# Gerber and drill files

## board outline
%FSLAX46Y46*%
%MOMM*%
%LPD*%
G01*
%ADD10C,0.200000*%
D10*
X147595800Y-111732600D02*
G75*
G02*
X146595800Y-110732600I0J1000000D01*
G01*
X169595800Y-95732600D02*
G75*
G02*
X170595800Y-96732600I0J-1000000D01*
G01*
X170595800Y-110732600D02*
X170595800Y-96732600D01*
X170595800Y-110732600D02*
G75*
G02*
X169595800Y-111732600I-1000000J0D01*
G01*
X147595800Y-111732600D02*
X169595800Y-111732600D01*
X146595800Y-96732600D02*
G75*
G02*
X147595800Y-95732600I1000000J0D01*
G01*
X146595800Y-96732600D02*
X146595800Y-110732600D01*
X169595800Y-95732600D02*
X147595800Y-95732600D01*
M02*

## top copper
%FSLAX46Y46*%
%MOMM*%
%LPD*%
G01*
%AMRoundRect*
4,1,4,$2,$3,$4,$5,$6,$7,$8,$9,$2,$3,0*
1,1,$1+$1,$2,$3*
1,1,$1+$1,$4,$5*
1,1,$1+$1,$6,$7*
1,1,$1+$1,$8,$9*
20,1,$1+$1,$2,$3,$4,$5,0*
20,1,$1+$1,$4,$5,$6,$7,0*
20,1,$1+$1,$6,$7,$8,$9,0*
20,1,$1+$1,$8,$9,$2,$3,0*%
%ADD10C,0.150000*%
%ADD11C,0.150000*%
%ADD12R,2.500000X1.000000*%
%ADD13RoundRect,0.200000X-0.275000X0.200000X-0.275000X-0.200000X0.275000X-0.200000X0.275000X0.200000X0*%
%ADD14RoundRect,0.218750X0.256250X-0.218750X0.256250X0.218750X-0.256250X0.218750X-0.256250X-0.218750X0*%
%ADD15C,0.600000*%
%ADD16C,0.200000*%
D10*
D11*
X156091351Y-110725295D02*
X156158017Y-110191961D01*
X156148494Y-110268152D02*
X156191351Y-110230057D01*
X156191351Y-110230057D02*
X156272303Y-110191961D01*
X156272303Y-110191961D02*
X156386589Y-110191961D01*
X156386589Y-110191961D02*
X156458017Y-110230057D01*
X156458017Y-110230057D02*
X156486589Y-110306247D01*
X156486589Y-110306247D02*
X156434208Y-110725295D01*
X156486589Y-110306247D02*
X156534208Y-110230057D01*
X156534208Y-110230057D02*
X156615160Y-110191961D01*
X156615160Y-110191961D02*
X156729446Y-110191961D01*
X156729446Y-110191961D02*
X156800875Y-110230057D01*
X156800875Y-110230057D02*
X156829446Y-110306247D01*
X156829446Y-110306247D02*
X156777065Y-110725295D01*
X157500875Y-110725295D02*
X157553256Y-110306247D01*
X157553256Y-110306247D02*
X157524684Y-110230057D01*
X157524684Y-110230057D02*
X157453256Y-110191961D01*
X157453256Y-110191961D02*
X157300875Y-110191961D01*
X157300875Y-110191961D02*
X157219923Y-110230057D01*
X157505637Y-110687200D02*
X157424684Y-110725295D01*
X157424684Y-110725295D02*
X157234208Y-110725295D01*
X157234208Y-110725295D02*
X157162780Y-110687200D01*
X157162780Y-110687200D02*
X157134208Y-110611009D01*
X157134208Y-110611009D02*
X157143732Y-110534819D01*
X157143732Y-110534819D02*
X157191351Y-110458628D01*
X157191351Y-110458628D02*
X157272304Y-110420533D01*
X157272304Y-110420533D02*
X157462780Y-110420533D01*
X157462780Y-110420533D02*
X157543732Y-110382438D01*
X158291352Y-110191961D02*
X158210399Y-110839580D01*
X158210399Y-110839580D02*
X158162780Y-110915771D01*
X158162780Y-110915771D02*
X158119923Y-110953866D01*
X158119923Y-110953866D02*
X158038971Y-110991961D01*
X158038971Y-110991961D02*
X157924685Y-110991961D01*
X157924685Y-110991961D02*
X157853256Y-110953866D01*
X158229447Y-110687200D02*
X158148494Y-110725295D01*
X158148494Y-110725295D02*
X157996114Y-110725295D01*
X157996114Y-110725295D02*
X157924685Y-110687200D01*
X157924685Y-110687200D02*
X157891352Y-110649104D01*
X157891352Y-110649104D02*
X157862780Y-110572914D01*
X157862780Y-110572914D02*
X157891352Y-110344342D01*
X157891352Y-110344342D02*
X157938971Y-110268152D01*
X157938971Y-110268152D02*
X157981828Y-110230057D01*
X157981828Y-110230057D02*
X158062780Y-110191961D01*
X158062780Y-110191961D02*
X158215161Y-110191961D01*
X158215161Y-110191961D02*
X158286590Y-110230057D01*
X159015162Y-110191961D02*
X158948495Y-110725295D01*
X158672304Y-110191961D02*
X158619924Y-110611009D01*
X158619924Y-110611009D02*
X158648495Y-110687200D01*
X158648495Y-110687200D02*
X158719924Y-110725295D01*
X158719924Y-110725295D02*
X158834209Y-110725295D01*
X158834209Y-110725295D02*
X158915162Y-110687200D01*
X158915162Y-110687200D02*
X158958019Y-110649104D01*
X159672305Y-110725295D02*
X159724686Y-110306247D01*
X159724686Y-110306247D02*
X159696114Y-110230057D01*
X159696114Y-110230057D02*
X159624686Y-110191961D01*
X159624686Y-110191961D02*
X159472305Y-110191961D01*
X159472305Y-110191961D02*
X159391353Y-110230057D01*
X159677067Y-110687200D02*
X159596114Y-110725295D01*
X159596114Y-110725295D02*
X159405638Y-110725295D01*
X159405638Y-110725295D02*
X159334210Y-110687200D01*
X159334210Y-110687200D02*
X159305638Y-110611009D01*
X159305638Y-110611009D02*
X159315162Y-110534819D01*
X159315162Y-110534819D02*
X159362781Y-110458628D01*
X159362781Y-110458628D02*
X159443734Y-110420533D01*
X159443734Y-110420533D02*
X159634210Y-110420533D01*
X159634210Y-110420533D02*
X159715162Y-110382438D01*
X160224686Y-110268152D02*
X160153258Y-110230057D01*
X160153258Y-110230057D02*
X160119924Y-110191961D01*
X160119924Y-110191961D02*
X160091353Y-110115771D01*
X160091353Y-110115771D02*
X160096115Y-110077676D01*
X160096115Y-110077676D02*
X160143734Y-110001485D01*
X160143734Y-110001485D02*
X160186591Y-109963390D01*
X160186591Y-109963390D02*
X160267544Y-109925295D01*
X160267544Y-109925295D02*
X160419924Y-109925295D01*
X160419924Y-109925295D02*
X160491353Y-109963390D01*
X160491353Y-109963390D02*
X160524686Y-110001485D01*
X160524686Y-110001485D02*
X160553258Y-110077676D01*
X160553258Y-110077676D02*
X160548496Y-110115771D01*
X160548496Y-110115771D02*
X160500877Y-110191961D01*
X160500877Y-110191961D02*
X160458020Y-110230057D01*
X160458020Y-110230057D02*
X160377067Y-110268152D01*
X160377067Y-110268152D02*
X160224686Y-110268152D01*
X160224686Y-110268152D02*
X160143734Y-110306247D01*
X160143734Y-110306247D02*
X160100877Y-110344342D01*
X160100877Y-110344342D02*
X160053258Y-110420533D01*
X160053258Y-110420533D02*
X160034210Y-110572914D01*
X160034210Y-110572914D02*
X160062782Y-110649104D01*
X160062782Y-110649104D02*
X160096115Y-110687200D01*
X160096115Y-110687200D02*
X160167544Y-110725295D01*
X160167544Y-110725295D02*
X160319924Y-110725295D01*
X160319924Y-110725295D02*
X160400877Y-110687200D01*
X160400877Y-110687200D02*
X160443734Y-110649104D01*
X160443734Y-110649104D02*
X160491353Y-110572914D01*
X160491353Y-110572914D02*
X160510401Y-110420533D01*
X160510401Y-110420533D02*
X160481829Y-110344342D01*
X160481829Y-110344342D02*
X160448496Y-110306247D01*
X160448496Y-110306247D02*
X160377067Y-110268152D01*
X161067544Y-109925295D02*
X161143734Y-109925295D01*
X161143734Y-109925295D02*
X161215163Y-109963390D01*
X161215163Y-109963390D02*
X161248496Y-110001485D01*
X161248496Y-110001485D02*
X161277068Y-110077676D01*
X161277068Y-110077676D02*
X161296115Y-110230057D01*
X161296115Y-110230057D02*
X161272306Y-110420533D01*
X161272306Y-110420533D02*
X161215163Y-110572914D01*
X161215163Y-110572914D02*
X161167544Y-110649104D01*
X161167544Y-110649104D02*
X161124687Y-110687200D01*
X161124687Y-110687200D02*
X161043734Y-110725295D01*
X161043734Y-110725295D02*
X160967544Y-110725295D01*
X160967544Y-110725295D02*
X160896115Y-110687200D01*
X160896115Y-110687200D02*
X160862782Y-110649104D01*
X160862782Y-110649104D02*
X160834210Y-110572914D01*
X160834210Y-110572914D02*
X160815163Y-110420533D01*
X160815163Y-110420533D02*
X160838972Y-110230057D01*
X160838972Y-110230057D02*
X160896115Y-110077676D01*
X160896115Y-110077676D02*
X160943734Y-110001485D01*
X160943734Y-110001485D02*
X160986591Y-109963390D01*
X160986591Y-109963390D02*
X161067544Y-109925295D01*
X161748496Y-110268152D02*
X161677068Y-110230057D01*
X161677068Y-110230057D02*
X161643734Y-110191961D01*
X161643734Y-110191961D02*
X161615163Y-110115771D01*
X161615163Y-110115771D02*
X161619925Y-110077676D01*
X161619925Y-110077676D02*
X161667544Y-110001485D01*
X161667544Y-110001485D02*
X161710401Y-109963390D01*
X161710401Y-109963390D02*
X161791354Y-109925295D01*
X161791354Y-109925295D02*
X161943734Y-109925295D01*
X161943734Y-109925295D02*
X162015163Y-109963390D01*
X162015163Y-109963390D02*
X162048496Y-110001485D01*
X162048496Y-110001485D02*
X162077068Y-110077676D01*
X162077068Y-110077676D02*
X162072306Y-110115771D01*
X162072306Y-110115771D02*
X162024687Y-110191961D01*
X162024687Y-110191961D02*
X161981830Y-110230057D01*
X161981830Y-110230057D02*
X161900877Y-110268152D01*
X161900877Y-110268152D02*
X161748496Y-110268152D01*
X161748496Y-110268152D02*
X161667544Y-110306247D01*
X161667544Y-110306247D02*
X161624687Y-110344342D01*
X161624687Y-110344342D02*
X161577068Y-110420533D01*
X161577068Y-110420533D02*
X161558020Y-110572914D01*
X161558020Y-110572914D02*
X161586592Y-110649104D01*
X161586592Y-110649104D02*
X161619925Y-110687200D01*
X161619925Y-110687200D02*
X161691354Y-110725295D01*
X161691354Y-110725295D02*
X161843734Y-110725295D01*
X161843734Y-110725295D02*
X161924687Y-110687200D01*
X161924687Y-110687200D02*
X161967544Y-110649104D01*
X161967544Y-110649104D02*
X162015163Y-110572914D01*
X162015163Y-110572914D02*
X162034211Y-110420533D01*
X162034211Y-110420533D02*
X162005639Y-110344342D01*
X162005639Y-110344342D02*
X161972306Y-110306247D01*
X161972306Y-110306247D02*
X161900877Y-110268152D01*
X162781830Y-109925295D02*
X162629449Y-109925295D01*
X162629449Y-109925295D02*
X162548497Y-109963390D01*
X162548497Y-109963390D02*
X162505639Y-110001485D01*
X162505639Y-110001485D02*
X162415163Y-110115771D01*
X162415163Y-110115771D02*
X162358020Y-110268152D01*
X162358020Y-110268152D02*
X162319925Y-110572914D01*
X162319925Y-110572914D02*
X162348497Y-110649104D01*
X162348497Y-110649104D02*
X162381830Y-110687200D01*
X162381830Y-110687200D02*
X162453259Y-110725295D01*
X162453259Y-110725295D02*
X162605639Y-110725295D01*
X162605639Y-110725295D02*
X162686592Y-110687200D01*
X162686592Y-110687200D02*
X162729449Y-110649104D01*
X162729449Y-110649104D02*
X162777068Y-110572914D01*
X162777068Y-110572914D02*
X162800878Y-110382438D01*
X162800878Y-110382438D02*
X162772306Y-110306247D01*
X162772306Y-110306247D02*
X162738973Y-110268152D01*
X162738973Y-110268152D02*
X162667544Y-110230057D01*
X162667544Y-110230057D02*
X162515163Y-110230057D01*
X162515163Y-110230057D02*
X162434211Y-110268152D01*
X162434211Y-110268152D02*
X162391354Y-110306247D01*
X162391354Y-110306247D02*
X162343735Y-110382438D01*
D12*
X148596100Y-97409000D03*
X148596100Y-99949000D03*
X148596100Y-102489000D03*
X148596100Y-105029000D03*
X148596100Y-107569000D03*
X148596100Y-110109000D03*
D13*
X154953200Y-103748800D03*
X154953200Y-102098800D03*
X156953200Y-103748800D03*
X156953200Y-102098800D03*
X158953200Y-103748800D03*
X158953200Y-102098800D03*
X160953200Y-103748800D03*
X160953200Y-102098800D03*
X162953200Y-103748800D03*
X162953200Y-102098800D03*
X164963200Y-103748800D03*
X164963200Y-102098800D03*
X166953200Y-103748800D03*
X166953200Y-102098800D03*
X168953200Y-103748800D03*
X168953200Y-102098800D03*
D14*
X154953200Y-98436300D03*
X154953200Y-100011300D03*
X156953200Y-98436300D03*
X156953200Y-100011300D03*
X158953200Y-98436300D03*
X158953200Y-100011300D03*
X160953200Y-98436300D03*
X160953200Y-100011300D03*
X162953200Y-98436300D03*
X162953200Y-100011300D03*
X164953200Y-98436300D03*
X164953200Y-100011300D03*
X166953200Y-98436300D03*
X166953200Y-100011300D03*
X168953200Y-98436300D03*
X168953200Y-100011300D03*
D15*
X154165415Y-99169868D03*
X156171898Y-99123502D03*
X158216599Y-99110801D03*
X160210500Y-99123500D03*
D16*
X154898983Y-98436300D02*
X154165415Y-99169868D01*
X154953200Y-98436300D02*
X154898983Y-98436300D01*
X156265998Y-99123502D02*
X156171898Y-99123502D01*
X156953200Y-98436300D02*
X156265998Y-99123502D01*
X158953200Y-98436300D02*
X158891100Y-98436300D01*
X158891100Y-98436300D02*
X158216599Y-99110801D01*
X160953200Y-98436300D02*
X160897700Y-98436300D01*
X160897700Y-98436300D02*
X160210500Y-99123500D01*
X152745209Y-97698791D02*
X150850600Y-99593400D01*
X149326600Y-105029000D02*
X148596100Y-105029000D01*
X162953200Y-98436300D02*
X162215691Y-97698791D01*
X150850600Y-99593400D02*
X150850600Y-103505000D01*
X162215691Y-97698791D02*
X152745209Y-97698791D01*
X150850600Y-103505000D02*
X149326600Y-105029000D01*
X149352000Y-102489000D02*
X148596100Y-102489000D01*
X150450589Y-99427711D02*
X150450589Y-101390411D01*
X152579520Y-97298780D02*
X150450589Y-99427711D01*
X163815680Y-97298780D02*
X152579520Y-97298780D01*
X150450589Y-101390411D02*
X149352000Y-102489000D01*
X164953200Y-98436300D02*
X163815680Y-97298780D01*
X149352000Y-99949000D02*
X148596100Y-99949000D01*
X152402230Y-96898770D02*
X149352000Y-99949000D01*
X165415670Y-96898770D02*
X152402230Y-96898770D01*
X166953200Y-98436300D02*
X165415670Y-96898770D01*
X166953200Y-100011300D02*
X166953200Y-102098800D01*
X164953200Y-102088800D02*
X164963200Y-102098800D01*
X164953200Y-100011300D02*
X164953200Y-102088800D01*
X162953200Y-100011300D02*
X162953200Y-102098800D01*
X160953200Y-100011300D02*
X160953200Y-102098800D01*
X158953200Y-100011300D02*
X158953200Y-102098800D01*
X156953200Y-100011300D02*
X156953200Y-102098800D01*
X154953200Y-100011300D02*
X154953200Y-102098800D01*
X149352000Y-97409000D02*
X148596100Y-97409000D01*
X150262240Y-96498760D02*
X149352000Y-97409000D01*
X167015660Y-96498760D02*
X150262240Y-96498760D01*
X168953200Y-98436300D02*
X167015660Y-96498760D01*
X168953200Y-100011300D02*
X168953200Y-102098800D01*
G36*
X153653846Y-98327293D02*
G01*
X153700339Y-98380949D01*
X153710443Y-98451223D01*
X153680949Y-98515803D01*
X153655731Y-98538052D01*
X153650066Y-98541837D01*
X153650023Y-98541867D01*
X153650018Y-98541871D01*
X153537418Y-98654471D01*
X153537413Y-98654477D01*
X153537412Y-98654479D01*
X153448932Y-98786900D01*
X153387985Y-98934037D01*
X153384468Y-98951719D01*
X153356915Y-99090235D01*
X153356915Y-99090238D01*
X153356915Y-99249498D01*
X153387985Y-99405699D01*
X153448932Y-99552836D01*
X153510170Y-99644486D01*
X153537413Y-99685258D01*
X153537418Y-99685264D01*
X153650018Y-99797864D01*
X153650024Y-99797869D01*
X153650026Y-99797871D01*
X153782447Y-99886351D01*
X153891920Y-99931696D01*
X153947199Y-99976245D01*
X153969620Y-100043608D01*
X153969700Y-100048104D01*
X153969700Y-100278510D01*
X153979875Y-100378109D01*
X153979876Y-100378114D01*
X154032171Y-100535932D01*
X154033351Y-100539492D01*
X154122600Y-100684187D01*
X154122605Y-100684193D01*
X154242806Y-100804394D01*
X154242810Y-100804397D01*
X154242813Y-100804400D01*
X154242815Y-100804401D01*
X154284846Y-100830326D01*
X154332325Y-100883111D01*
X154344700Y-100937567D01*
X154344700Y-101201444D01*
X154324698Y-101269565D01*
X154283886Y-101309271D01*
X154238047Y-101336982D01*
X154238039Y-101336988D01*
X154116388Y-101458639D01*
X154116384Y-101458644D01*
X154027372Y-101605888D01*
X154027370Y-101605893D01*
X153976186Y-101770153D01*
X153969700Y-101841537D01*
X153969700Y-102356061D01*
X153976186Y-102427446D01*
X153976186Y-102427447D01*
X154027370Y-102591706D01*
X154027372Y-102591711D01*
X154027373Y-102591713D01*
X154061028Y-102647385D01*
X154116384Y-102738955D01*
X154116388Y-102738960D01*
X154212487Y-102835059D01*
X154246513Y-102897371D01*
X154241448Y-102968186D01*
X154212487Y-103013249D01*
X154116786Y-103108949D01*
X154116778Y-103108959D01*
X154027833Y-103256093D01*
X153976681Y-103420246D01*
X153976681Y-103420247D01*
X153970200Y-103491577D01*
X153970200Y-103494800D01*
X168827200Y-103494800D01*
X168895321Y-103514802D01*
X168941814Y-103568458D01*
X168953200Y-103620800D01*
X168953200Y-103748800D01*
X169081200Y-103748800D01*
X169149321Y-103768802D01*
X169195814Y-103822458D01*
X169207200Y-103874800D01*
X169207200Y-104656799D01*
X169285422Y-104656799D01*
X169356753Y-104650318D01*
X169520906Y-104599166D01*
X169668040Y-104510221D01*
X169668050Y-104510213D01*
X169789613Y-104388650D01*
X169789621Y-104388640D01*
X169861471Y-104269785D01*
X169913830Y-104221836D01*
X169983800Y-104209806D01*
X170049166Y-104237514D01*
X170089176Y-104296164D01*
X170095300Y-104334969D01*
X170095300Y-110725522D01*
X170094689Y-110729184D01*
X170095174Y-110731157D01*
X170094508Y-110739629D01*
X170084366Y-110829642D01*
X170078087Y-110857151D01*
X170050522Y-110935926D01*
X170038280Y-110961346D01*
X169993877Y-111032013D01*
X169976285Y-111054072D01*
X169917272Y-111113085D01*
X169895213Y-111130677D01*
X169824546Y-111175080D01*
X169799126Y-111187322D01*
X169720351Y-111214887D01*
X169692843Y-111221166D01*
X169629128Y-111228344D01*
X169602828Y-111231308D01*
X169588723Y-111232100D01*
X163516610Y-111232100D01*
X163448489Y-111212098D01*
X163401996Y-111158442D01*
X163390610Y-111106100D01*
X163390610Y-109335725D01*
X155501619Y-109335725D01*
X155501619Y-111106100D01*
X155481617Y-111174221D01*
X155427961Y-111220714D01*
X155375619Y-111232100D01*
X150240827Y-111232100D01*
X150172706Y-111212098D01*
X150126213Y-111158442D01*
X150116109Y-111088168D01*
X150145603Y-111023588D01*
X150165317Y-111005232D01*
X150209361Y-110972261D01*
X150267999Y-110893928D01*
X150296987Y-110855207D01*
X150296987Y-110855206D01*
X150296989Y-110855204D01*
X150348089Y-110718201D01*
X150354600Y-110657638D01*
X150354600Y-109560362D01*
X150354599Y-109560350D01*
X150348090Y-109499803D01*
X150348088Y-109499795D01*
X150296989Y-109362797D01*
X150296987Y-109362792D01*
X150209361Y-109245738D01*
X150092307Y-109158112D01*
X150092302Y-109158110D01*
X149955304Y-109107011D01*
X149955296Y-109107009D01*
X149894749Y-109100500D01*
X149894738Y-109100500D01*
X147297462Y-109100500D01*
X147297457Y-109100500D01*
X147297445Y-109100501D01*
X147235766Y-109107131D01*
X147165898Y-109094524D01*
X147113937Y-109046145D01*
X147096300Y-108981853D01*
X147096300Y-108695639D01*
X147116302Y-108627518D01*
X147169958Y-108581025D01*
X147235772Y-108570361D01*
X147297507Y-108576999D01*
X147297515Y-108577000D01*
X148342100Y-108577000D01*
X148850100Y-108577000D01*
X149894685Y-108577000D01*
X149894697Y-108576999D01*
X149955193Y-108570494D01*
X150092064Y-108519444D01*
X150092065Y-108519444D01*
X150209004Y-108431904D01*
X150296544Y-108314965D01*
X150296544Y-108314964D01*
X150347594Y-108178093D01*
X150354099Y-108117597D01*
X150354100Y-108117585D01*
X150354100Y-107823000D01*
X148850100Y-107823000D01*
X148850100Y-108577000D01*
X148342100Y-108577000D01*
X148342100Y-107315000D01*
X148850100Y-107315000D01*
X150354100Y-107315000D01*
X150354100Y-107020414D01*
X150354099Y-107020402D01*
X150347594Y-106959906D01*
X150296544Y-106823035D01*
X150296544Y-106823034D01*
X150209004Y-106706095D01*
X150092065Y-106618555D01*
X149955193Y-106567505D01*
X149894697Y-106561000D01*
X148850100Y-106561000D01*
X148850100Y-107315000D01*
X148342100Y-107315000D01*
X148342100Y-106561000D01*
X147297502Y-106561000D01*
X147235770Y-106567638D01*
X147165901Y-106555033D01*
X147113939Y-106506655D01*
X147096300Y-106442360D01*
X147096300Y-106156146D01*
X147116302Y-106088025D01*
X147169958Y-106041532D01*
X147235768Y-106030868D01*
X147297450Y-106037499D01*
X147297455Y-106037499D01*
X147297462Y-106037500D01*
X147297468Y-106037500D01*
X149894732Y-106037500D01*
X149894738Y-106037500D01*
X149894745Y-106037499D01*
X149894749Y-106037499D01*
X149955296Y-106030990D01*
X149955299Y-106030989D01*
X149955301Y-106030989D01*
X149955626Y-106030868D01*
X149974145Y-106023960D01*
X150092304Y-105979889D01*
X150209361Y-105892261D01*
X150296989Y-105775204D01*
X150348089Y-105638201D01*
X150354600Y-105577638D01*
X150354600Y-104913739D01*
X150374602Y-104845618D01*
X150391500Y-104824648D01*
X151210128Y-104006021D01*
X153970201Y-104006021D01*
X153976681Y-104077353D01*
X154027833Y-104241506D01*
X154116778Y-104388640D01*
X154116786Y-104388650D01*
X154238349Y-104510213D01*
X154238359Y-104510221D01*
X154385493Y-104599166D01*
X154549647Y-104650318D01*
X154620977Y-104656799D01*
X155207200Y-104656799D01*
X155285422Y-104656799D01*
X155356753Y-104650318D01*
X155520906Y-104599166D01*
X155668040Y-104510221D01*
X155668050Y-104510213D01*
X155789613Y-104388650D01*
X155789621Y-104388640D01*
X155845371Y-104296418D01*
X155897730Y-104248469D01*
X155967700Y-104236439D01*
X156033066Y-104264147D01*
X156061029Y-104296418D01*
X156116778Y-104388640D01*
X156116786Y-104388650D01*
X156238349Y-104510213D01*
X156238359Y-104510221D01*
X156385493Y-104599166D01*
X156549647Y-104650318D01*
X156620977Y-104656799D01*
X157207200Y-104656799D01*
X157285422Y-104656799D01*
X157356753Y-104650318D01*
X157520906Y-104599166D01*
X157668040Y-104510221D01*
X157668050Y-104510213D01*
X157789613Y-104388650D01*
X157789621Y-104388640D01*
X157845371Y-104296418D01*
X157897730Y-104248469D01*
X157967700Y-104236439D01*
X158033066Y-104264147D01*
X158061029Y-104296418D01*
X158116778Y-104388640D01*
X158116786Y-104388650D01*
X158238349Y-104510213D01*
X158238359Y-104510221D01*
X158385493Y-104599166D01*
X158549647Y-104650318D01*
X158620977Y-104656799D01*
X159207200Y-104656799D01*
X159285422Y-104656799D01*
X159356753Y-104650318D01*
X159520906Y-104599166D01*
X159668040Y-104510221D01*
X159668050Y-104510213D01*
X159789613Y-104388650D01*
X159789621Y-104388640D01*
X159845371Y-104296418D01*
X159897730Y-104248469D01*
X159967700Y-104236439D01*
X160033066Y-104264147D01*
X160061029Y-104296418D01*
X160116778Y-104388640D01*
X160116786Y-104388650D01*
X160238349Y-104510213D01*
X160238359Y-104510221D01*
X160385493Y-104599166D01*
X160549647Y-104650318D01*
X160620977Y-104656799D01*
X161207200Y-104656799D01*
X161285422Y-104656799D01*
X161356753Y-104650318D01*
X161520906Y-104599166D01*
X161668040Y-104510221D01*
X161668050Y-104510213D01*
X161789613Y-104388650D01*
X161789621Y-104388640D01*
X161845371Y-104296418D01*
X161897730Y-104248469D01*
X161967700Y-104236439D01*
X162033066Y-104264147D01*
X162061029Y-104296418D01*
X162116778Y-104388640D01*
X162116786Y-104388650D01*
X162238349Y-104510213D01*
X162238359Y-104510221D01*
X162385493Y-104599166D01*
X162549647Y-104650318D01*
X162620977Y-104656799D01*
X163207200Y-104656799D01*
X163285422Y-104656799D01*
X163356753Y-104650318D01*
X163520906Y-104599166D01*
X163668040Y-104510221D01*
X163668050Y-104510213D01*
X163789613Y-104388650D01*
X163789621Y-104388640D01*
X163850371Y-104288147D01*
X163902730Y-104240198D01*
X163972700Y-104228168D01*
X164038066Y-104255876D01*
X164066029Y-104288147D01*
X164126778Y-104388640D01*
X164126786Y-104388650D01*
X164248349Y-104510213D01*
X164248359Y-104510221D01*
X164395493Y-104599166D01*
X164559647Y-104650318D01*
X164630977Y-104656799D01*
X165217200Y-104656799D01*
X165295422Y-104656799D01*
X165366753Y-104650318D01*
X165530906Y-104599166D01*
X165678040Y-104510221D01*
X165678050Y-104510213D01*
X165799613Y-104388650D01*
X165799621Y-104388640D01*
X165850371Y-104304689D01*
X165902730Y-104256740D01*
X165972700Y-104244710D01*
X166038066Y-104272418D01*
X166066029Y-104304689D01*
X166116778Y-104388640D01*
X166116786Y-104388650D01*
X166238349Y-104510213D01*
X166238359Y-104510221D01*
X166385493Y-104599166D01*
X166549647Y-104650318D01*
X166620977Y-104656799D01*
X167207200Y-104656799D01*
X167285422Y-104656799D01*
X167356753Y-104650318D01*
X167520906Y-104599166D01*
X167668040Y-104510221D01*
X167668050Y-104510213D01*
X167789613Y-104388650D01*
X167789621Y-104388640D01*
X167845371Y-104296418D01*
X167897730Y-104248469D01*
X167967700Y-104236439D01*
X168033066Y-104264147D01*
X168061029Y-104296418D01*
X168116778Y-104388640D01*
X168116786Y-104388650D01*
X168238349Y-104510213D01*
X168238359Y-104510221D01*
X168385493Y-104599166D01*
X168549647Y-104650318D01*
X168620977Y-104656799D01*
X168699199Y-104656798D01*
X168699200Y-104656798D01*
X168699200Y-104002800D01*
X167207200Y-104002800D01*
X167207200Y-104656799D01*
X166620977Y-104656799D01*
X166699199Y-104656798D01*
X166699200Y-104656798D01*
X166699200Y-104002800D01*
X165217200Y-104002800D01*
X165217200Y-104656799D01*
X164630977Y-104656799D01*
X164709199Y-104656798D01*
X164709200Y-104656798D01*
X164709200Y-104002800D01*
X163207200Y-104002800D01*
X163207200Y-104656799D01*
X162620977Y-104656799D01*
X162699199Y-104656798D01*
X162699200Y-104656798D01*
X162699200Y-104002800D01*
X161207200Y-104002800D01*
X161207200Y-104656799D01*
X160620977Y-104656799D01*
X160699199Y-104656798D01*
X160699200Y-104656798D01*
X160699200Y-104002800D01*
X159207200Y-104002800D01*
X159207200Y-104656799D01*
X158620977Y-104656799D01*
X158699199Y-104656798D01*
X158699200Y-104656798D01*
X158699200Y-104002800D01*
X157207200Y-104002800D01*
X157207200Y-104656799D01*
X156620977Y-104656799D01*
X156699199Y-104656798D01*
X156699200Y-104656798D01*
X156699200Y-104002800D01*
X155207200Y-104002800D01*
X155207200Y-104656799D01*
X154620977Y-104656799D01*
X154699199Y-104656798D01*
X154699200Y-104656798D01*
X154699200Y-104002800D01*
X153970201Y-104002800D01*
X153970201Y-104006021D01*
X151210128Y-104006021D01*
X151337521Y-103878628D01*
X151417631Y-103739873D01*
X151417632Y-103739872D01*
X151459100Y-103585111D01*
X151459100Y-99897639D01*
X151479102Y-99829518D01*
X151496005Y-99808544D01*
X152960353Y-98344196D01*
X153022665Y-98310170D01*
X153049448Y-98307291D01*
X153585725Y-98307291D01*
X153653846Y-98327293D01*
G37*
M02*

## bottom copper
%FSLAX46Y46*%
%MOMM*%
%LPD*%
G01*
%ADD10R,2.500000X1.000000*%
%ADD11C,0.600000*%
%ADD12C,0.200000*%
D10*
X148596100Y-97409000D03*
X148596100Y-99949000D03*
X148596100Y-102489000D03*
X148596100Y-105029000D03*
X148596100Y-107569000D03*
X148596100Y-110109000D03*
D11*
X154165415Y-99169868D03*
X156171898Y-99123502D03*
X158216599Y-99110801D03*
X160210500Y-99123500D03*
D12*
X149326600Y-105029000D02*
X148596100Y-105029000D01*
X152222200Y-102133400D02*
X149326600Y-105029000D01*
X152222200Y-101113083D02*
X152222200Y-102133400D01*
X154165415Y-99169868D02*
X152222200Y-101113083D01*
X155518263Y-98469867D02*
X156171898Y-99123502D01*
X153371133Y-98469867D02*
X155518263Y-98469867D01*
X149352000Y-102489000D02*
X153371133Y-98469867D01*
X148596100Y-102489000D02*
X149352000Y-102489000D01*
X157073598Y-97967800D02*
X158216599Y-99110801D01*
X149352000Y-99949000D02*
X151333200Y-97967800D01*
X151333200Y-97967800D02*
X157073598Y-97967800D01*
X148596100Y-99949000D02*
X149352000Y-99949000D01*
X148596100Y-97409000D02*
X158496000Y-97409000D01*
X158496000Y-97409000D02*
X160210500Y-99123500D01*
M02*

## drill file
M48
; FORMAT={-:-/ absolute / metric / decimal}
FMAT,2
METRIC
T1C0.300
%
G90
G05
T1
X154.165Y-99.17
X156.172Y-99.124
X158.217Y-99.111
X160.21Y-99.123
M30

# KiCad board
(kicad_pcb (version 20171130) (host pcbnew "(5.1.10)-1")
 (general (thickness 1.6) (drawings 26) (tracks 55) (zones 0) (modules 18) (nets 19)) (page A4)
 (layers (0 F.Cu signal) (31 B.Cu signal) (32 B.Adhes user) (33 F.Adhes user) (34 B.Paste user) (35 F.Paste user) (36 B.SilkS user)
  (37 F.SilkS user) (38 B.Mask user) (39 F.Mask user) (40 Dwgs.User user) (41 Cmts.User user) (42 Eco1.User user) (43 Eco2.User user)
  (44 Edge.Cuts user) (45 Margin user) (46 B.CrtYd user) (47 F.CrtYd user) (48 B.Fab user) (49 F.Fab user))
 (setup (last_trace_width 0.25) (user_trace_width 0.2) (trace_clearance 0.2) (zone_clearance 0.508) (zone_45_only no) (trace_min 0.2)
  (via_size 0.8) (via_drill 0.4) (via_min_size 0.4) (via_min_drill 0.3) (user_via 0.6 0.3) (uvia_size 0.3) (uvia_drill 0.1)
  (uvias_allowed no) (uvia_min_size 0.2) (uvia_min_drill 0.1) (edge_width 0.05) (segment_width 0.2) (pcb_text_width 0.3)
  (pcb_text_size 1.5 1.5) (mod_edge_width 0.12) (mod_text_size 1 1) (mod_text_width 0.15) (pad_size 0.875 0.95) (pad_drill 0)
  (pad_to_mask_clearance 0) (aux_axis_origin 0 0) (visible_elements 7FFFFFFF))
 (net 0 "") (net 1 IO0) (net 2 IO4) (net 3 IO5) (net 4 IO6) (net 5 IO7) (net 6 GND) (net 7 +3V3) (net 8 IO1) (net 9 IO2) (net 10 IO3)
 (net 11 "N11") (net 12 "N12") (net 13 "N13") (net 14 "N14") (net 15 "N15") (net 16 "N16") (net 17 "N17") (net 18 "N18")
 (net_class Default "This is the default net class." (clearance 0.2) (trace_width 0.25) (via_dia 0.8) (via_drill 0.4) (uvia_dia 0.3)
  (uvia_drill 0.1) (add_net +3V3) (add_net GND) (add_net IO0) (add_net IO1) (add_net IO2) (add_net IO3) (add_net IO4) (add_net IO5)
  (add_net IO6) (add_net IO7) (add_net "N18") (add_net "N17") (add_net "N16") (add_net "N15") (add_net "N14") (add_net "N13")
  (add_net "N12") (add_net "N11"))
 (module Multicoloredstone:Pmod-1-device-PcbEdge (layer F.Cu) (at 146.5961 103.759)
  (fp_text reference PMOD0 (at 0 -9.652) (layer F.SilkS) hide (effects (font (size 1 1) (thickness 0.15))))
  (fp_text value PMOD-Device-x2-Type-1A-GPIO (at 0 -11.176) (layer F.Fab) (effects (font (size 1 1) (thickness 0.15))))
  (pad 1 smd rect (at 2 -6.35 90) (size 1 2.5) (layers F.Cu F.Paste F.Mask) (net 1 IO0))
  (pad 7 smd rect (at 2 -6.35 90) (size 1 2.5) (layers B.Cu B.Paste B.Mask) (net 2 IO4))
  (pad 8 smd rect (at 2 -3.81 90) (size 1 2.5) (layers B.Cu B.Paste B.Mask) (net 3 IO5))
  (pad 9 smd rect (at 2 -1.27 90) (size 1 2.5) (layers B.Cu B.Paste B.Mask) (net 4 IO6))
  (pad 10 smd rect (at 2 1.27 90) (size 1 2.5) (layers B.Cu B.Paste B.Mask) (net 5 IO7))
  (pad 11 smd rect (at 2 3.81 90) (size 1 2.5) (layers B.Cu B.Paste B.Mask) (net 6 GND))
  (pad 12 smd rect (at 2 6.35 90) (size 1 2.5) (layers B.Cu B.Paste B.Mask) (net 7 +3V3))
  (pad 2 smd rect (at 2 -3.81 90) (size 1 2.5) (layers F.Cu F.Paste F.Mask) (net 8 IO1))
  (pad 3 smd rect (at 2 -1.27 90) (size 1 2.5) (layers F.Cu F.Paste F.Mask) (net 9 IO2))
  (pad 4 smd rect (at 2 1.27 90) (size 1 2.5) (layers F.Cu F.Paste F.Mask) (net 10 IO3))
  (pad 5 smd rect (at 2 3.81 90) (size 1 2.5) (layers F.Cu F.Paste F.Mask) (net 6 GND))
  (pad 6 smd rect (at 2 6.35 90) (size 1 2.5) (layers F.Cu F.Paste F.Mask) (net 7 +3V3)))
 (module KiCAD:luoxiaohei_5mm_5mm (layer F.Cu) (at 167.5384 108.458)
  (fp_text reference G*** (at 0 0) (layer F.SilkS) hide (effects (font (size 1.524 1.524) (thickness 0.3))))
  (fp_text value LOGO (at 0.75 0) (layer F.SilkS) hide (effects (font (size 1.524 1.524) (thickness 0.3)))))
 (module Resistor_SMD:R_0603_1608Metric (layer F.Cu) (at 154.9532 102.9238 270)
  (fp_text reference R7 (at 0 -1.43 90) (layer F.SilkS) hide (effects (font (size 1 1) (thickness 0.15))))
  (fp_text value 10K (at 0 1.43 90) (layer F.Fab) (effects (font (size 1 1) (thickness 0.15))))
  (pad 2 smd roundrect (at 0.825 0 270) (size 0.8 0.95) (layers F.Cu F.Paste F.Mask) (roundrect_rratio 0.25) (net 6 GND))
  (pad 1 smd roundrect (at -0.825 0 270) (size 0.8 0.95) (layers F.Cu F.Paste F.Mask) (roundrect_rratio 0.25) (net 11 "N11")))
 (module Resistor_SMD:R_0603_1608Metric (layer F.Cu) (at 156.9532 102.9238 270)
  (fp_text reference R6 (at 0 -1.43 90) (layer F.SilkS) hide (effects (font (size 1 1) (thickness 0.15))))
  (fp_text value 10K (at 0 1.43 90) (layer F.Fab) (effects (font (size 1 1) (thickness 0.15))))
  (pad 2 smd roundrect (at 0.825 0 270) (size 0.8 0.95) (layers F.Cu F.Paste F.Mask) (roundrect_rratio 0.25) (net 6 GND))
  (pad 1 smd roundrect (at -0.825 0 270) (size 0.8 0.95) (layers F.Cu F.Paste F.Mask) (roundrect_rratio 0.25) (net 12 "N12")))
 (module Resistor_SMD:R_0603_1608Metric (layer F.Cu) (at 158.9532 102.9238 270)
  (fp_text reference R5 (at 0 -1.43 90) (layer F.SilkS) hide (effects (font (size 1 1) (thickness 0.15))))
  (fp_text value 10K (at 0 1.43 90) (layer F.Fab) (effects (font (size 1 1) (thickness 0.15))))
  (pad 2 smd roundrect (at 0.825 0 270) (size 0.8 0.95) (layers F.Cu F.Paste F.Mask) (roundrect_rratio 0.25) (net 6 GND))
  (pad 1 smd roundrect (at -0.825 0 270) (size 0.8 0.95) (layers F.Cu F.Paste F.Mask) (roundrect_rratio 0.25) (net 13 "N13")))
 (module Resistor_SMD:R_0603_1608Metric (layer F.Cu) (at 160.9532 102.9238 270)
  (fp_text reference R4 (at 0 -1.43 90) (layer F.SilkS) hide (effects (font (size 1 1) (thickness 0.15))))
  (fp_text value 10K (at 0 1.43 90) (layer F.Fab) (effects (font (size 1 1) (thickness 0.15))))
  (pad 2 smd roundrect (at 0.825 0 270) (size 0.8 0.95) (layers F.Cu F.Paste F.Mask) (roundrect_rratio 0.25) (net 6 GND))
  (pad 1 smd roundrect (at -0.825 0 270) (size 0.8 0.95) (layers F.Cu F.Paste F.Mask) (roundrect_rratio 0.25) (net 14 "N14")))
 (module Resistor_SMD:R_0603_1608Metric (layer F.Cu) (at 162.9532 102.9238 270)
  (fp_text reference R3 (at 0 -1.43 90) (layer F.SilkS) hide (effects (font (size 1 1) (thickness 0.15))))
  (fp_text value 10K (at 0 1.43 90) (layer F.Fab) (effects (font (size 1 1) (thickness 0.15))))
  (pad 2 smd roundrect (at 0.825 0 270) (size 0.8 0.95) (layers F.Cu F.Paste F.Mask) (roundrect_rratio 0.25) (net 6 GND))
  (pad 1 smd roundrect (at -0.825 0 270) (size 0.8 0.95) (layers F.Cu F.Paste F.Mask) (roundrect_rratio 0.25) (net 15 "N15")))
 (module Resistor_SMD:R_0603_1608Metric (layer F.Cu) (at 164.9632 102.9238 270)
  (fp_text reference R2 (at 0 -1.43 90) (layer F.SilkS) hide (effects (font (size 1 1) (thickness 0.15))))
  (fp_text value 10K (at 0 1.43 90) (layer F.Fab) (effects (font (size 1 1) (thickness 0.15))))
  (pad 2 smd roundrect (at 0.825 0 270) (size 0.8 0.95) (layers F.Cu F.Paste F.Mask) (roundrect_rratio 0.25) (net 6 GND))
  (pad 1 smd roundrect (at -0.825 0 270) (size 0.8 0.95) (layers F.Cu F.Paste F.Mask) (roundrect_rratio 0.25) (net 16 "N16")))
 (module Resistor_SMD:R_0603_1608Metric (layer F.Cu) (at 166.9532 102.9238 270)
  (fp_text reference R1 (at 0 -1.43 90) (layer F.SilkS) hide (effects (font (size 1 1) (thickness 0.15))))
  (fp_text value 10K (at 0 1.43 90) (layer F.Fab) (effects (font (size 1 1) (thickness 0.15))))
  (pad 2 smd roundrect (at 0.825 0 270) (size 0.8 0.95) (layers F.Cu F.Paste F.Mask) (roundrect_rratio 0.25) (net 6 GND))
  (pad 1 smd roundrect (at -0.825 0 270) (size 0.8 0.95) (layers F.Cu F.Paste F.Mask) (roundrect_rratio 0.25) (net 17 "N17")))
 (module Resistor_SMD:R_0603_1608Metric (layer F.Cu) (at 168.9532 102.9238 270)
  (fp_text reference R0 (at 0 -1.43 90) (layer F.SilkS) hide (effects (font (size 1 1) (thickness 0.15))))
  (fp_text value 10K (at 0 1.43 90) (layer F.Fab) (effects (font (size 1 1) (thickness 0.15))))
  (pad 2 smd roundrect (at 0.825 0 270) (size 0.8 0.95) (layers F.Cu F.Paste F.Mask) (roundrect_rratio 0.25) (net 6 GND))
  (pad 1 smd roundrect (at -0.825 0 270) (size 0.8 0.95) (layers F.Cu F.Paste F.Mask) (roundrect_rratio 0.25) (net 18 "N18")))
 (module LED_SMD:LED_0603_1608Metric (layer F.Cu) (at 154.9532 99.2238 90)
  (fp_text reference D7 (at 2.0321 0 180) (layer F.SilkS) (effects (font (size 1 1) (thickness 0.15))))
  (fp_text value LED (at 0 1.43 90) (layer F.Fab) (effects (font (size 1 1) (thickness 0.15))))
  (pad 2 smd roundrect (at 0.7875 0 90) (size 0.875 0.95) (layers F.Cu F.Paste F.Mask) (roundrect_rratio 0.25) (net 5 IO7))
  (pad 1 smd roundrect (at -0.7875 0 90) (size 0.875 0.95) (layers F.Cu F.Paste F.Mask) (roundrect_rratio 0.25) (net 11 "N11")))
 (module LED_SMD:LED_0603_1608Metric (layer F.Cu) (at 156.9532 99.2238 90)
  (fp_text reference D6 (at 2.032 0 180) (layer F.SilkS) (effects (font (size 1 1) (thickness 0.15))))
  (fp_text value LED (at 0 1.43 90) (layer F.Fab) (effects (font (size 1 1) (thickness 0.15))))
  (pad 2 smd roundrect (at 0.7875 0 90) (size 0.875 0.95) (layers F.Cu F.Paste F.Mask) (roundrect_rratio 0.25) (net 4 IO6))
  (pad 1 smd roundrect (at -0.7875 0 90) (size 0.875 0.95) (layers F.Cu F.Paste F.Mask) (roundrect_rratio 0.25) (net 12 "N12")))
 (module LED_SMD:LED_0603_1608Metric (layer F.Cu) (at 158.9532 99.2238 90)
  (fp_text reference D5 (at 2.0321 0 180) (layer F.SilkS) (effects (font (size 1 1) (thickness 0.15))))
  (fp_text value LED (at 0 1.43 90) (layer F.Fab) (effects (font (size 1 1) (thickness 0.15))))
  (pad 2 smd roundrect (at 0.7875 0 90) (size 0.875 0.95) (layers F.Cu F.Paste F.Mask) (roundrect_rratio 0.25) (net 3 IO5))
  (pad 1 smd roundrect (at -0.7875 0 90) (size 0.875 0.95) (layers F.Cu F.Paste F.Mask) (roundrect_rratio 0.25) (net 13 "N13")))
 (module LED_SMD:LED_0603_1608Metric (layer F.Cu) (at 160.9532 99.2238 90)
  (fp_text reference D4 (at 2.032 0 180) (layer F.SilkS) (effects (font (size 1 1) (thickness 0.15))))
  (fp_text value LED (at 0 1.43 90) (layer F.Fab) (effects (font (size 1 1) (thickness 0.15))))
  (pad 2 smd roundrect (at 0.7875 0 90) (size 0.875 0.95) (layers F.Cu F.Paste F.Mask) (roundrect_rratio 0.25) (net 2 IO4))
  (pad 1 smd roundrect (at -0.7875 0 90) (size 0.875 0.95) (layers F.Cu F.Paste F.Mask) (roundrect_rratio 0.25) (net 14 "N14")))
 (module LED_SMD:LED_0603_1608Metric (layer F.Cu) (at 162.9532 99.2238 90)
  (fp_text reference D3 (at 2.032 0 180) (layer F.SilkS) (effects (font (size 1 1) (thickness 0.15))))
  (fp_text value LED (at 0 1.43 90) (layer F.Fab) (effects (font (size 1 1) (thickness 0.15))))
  (pad 2 smd roundrect (at 0.7875 0 90) (size 0.875 0.95) (layers F.Cu F.Paste F.Mask) (roundrect_rratio 0.25) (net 10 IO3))
  (pad 1 smd roundrect (at -0.7875 0 90) (size 0.875 0.95) (layers F.Cu F.Paste F.Mask) (roundrect_rratio 0.25) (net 15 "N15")))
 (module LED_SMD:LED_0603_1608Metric (layer F.Cu) (at 164.9532 99.2238 90)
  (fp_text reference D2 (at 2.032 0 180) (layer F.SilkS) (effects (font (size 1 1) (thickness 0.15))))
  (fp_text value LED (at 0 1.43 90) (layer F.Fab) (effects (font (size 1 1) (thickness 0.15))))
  (pad 2 smd roundrect (at 0.7875 0 90) (size 0.875 0.95) (layers F.Cu F.Paste F.Mask) (roundrect_rratio 0.25) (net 9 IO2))
  (pad 1 smd roundrect (at -0.7875 0 90) (size 0.875 0.95) (layers F.Cu F.Paste F.Mask) (roundrect_rratio 0.25) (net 16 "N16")))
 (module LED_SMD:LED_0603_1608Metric (layer F.Cu) (at 166.9532 99.2238 90)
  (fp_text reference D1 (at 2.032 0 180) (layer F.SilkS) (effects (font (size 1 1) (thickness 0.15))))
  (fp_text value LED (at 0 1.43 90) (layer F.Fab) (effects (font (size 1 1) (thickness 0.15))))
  (pad 2 smd roundrect (at 0.7875 0 90) (size 0.875 0.95) (layers F.Cu F.Paste F.Mask) (roundrect_rratio 0.25) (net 8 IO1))
  (pad 1 smd roundrect (at -0.7875 0 90) (size 0.875 0.95) (layers F.Cu F.Paste F.Mask) (roundrect_rratio 0.25) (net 17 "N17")))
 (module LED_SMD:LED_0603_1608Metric (layer F.Cu) (at 168.9532 99.2238 90)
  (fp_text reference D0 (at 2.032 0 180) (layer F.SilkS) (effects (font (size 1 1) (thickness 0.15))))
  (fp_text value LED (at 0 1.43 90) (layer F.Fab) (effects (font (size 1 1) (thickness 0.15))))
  (pad 2 smd roundrect (at 0.7875 0 90) (size 0.875 0.95) (layers F.Cu F.Paste F.Mask) (roundrect_rratio 0.25) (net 1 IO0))
  (pad 1 smd roundrect (at -0.7875 0 90) (size 0.875 0.95) (layers F.Cu F.Paste F.Mask) (roundrect_rratio 0.25) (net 18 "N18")))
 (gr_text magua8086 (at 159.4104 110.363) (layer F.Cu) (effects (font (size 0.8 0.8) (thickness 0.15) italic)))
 (gr_arc (start 147.5958 110.7326) (end 146.5958 110.7326) (angle -90) (layer Edge.Cuts) (width 0.2))
 (gr_arc (start 169.5958 96.7326) (end 170.5958 96.7326) (angle -90) (layer Edge.Cuts) (width 0.2))
 (gr_line (start 170.5958 110.7326) (end 170.5958 96.7326) (layer Edge.Cuts) (width 0.2))
 (gr_arc (start 169.5958 110.7326) (end 169.5958 111.7326) (angle -90) (layer Edge.Cuts) (width 0.2))
 (gr_line (start 147.5958 111.7326) (end 169.5958 111.7326) (layer Edge.Cuts) (width 0.2))
 (gr_arc (start 147.5958 96.7326) (end 147.5958 95.7326) (angle -90) (layer Edge.Cuts) (width 0.2))
 (gr_line (start 146.5958 96.7326) (end 146.5958 110.7326) (layer Edge.Cuts) (width 0.2))
 (gr_line (start 169.5958 95.7326) (end 147.5958 95.7326) (layer Edge.Cuts) (width 0.2))
 (segment (start 154.898983 98.4363) (end 154.165415 99.169868) (width 0.2) (layer F.Cu) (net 5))
 (segment (start 154.9532 98.4363) (end 154.898983 98.4363) (width 0.2) (layer F.Cu) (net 5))
 (via (at 154.165415 99.169868) (size 0.6) (drill 0.3) (layers F.Cu B.Cu) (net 5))
 (segment (start 149.3266 105.029) (end 148.5961 105.029) (width 0.2) (layer B.Cu) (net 5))
 (segment (start 152.2222 102.1334) (end 149.3266 105.029) (width 0.2) (layer B.Cu) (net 5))
 (segment (start 152.2222 101.113083) (end 152.2222 102.1334) (width 0.2) (layer B.Cu) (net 5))
 (segment (start 154.165415 99.169868) (end 152.2222 101.113083) (width 0.2) (layer B.Cu) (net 5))
 (segment (start 156.265998 99.123502) (end 156.171898 99.123502) (width 0.2) (layer F.Cu) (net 4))
 (segment (start 156.9532 98.4363) (end 156.265998 99.123502) (width 0.2) (layer F.Cu) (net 4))
 (via (at 156.171898 99.123502) (size 0.6) (drill 0.3) (layers F.Cu B.Cu) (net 4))
 (segment (start 155.518263 98.469867) (end 156.171898 99.123502) (width 0.2) (layer B.Cu) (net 4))
 (segment (start 153.371133 98.469867) (end 155.518263 98.469867) (width 0.2) (layer B.Cu) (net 4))
 (segment (start 149.352 102.489) (end 153.371133 98.469867) (width 0.2) (layer B.Cu) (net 4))
 (segment (start 148.5961 102.489) (end 149.352 102.489) (width 0.2) (layer B.Cu) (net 4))
 (via (at 158.216599 99.110801) (size 0.6) (drill 0.3) (layers F.Cu B.Cu) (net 3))
 (segment (start 158.9532 98.4363) (end 158.8911 98.4363) (width 0.2) (layer F.Cu) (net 3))
 (segment (start 158.8911 98.4363) (end 158.216599 99.110801) (width 0.2) (layer F.Cu) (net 3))
 (segment (start 157.073598 97.9678) (end 158.216599 99.110801) (width 0.2) (layer B.Cu) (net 3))
 (segment (start 149.352 99.949) (end 151.3332 97.9678) (width 0.2) (layer B.Cu) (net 3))
 (segment (start 151.3332 97.9678) (end 157.073598 97.9678) (width 0.2) (layer B.Cu) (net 3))
 (segment (start 148.5961 99.949) (end 149.352 99.949) (width 0.2) (layer B.Cu) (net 3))
 (via (at 160.2105 99.1235) (size 0.6) (drill 0.3) (layers F.Cu B.Cu) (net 2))
 (segment (start 160.9532 98.4363) (end 160.8977 98.4363) (width 0.2) (layer F.Cu) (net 2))
 (segment (start 160.8977 98.4363) (end 160.2105 99.1235) (width 0.2) (layer F.Cu) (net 2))
 (segment (start 148.5961 97.409) (end 158.496 97.409) (width 0.2) (layer B.Cu) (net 2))
 (segment (start 158.496 97.409) (end 160.2105 99.1235) (width 0.2) (layer B.Cu) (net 2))
 (segment (start 152.745209 97.698791) (end 150.8506 99.5934) (width 0.2) (layer F.Cu) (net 10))
 (segment (start 149.3266 105.029) (end 148.5961 105.029) (width 0.2) (layer F.Cu) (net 10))
 (segment (start 162.9532 98.4363) (end 162.215691 97.698791) (width 0.2) (layer F.Cu) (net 10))
 (segment (start 150.8506 99.5934) (end 150.8506 103.505) (width 0.2) (layer F.Cu) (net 10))
 (segment (start 162.215691 97.698791) (end 152.745209 97.698791) (width 0.2) (layer F.Cu) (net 10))
 (segment (start 150.8506 103.505) (end 149.3266 105.029) (width 0.2) (layer F.Cu) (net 10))
 (segment (start 149.352 102.489) (end 148.5961 102.489) (width 0.2) (layer F.Cu) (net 9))
 (segment (start 150.450589 99.427711) (end 150.450589 101.390411) (width 0.2) (layer F.Cu) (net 9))
 (segment (start 152.57952 97.29878) (end 150.450589 99.427711) (width 0.2) (layer F.Cu) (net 9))
 (segment (start 163.81568 97.29878) (end 152.57952 97.29878) (width 0.2) (layer F.Cu) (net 9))
 (segment (start 150.450589 101.390411) (end 149.352 102.489) (width 0.2) (layer F.Cu) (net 9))
 (segment (start 164.9532 98.4363) (end 163.81568 97.29878) (width 0.2) (layer F.Cu) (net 9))
 (segment (start 149.352 99.949) (end 148.5961 99.949) (width 0.2) (layer F.Cu) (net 8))
 (segment (start 152.40223 96.89877) (end 149.352 99.949) (width 0.2) (layer F.Cu) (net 8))
 (segment (start 165.41567 96.89877) (end 152.40223 96.89877) (width 0.2) (layer F.Cu) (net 8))
 (segment (start 166.9532 98.4363) (end 165.41567 96.89877) (width 0.2) (layer F.Cu) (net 8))
 (segment (start 166.9532 100.0113) (end 166.9532 102.0988) (width 0.2) (layer F.Cu) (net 17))
 (segment (start 164.9532 102.0888) (end 164.9632 102.0988) (width 0.2) (layer F.Cu) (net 16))
 (segment (start 164.9532 100.0113) (end 164.9532 102.0888) (width 0.2) (layer F.Cu) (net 16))
 (segment (start 162.9532 100.0113) (end 162.9532 102.0988) (width 0.2) (layer F.Cu) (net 15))
 (segment (start 160.9532 100.0113) (end 160.9532 102.0988) (width 0.2) (layer F.Cu) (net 14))
 (segment (start 158.9532 100.0113) (end 158.9532 102.0988) (width 0.2) (layer F.Cu) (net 13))
 (segment (start 156.9532 100.0113) (end 156.9532 102.0988) (width 0.2) (layer F.Cu) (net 12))
 (segment (start 154.9532 100.0113) (end 154.9532 102.0988) (width 0.2) (layer F.Cu) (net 11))
 (segment (start 149.352 97.409) (end 148.5961 97.409) (width 0.2) (layer F.Cu) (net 1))
 (segment (start 150.26224 96.49876) (end 149.352 97.409) (width 0.2) (layer F.Cu) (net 1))
 (segment (start 167.01566 96.49876) (end 150.26224 96.49876) (width 0.2) (layer F.Cu) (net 1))
 (segment (start 168.9532 98.4363) (end 167.01566 96.49876) (width 0.2) (layer F.Cu) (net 1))
 (segment (start 168.9532 100.0113) (end 168.9532 102.0988) (width 0.2) (layer F.Cu) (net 18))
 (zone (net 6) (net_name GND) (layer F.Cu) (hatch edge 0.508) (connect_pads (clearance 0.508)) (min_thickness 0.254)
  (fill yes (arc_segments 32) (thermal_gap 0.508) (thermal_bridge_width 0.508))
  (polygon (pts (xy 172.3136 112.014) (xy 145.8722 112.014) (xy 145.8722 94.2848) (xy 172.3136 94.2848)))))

